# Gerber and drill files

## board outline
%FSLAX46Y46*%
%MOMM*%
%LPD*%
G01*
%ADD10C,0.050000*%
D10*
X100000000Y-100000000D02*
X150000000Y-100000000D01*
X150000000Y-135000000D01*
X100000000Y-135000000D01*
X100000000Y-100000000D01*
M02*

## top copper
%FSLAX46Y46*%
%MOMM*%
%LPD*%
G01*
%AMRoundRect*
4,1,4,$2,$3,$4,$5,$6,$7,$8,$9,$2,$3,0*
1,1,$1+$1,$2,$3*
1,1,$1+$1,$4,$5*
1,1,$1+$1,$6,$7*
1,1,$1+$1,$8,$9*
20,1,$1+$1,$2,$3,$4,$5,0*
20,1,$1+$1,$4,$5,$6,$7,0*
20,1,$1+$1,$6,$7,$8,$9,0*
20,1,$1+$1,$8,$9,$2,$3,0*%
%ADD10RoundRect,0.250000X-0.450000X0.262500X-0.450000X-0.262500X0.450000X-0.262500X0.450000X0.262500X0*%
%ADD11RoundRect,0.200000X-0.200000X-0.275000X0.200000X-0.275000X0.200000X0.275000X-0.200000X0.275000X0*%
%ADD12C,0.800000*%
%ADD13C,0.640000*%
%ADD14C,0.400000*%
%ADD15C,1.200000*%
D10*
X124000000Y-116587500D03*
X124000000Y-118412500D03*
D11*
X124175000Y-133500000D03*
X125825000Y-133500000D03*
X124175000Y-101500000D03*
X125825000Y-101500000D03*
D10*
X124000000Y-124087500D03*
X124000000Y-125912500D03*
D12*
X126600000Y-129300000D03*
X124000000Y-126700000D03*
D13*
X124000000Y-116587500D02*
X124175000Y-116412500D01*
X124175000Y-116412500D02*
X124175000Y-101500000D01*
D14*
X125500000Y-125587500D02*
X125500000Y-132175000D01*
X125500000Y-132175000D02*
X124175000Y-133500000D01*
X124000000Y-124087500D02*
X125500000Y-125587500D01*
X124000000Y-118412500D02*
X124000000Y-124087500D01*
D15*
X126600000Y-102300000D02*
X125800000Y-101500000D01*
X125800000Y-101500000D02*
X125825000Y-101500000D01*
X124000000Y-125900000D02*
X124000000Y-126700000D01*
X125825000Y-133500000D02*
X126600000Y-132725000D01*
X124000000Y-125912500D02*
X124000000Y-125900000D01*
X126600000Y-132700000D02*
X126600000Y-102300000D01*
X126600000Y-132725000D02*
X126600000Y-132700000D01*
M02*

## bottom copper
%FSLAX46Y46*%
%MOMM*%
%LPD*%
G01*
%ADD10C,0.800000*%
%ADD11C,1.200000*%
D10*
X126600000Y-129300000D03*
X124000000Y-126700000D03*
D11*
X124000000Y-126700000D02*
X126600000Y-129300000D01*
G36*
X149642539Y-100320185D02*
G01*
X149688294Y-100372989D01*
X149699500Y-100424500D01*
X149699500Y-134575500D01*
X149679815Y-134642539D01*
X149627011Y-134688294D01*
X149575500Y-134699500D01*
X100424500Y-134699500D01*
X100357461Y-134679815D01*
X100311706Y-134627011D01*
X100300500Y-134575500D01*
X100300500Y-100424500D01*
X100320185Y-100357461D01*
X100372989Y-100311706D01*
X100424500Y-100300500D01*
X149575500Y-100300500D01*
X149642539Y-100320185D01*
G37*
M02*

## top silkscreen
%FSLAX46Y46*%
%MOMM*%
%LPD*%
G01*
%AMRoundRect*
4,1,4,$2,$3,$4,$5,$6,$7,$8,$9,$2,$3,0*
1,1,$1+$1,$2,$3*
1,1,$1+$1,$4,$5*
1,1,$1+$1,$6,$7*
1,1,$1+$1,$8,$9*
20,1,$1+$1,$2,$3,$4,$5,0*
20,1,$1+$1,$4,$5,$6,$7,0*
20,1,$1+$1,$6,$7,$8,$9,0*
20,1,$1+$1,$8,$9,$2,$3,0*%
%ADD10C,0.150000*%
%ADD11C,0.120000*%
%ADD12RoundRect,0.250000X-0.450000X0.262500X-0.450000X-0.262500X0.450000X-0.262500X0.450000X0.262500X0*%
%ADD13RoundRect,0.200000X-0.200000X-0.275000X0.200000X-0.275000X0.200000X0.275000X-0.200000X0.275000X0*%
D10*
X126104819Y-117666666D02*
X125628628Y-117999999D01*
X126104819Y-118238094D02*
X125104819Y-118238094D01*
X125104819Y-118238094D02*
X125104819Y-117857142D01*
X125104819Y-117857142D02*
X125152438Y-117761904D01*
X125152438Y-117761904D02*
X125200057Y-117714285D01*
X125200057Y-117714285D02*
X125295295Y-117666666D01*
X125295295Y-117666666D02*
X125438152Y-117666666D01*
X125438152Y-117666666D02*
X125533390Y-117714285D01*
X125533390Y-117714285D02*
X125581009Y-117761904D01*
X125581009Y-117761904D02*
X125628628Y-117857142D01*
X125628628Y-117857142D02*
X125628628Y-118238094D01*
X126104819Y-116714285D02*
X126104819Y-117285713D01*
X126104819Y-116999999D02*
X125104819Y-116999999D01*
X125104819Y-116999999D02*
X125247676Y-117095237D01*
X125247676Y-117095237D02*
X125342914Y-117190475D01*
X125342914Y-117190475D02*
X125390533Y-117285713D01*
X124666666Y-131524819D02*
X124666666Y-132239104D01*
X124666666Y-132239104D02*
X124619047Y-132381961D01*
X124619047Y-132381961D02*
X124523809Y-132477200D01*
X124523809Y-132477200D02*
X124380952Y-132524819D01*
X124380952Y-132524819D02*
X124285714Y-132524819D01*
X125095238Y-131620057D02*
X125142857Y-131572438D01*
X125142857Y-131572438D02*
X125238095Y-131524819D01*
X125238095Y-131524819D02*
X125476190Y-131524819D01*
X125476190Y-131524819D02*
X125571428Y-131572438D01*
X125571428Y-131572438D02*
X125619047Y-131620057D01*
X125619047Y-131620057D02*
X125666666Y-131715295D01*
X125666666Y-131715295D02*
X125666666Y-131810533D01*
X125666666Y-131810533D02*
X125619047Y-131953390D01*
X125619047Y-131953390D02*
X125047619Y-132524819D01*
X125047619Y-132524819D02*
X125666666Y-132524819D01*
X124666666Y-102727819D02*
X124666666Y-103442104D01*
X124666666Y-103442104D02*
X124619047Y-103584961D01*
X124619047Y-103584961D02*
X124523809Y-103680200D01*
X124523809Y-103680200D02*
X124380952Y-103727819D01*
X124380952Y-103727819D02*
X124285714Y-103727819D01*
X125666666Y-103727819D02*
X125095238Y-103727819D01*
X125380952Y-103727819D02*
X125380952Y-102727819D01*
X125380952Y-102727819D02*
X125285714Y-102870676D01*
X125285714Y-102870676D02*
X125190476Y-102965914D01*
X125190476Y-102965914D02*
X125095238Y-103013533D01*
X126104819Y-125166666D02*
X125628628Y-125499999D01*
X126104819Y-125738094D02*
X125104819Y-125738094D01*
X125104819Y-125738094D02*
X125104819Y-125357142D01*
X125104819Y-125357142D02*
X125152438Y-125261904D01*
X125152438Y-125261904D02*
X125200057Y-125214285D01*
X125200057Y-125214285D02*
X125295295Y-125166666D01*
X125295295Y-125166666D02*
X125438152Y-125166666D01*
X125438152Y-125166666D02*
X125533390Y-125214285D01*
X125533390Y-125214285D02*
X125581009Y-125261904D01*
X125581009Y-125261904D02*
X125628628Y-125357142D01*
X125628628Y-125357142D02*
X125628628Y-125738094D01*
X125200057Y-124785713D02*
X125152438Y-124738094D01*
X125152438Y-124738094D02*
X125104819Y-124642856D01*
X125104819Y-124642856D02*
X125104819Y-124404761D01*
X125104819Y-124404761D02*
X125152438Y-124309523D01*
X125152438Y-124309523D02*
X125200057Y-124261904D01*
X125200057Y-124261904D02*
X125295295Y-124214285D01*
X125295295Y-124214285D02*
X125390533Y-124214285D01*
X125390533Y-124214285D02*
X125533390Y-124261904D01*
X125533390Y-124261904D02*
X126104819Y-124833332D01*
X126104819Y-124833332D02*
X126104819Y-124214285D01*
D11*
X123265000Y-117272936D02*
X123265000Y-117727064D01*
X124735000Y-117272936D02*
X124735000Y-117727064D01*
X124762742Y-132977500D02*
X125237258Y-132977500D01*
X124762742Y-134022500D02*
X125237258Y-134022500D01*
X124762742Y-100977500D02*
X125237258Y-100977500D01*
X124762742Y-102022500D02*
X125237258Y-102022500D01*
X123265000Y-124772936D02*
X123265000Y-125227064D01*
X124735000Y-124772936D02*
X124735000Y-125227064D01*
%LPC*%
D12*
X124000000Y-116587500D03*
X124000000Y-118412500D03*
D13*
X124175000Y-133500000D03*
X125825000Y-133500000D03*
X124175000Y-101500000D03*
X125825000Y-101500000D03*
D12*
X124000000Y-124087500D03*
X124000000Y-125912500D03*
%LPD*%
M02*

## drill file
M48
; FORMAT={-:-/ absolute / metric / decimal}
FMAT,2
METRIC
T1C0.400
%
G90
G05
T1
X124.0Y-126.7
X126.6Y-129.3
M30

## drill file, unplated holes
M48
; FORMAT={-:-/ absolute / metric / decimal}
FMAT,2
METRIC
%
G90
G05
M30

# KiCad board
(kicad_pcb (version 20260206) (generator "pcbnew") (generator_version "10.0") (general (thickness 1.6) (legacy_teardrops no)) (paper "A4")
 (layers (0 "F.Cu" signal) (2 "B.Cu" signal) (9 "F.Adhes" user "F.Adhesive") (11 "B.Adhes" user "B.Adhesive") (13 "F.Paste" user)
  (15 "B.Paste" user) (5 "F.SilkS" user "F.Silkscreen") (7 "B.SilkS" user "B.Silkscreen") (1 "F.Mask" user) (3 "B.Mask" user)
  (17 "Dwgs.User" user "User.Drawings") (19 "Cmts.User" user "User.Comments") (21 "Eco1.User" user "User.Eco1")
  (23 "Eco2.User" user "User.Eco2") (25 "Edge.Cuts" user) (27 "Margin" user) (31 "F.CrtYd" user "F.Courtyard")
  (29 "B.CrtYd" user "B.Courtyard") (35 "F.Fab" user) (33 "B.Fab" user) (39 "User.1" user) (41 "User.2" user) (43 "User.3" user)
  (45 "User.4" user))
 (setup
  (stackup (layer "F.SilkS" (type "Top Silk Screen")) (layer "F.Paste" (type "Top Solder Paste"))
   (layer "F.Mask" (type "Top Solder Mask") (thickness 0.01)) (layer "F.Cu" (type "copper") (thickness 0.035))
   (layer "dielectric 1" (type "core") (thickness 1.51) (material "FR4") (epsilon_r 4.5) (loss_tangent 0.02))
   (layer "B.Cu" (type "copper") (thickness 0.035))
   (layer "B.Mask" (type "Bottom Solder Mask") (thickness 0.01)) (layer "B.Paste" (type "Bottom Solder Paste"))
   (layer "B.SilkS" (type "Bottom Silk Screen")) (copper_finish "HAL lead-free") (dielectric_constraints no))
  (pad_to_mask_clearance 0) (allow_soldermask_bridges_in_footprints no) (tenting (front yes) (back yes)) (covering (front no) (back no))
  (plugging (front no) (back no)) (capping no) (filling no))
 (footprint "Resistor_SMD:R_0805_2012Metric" (layer "F.Cu") (at 124 117.5 -90)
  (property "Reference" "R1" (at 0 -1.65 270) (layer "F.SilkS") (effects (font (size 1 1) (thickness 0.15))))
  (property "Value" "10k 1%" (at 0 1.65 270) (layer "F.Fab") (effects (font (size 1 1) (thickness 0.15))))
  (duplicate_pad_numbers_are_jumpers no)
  (fp_line (start -0.227064 0.735) (end 0.227064 0.735) (stroke (width 0.12) (type solid)) (layer "F.SilkS"))
  (fp_line (start -0.227064 -0.735) (end 0.227064 -0.735) (stroke (width 0.12) (type solid)) (layer "F.SilkS"))
  (pad "1" smd roundrect (at -0.9125 0 270) (size 1.025 1.4) (layers "F.Cu" "F.Mask" "F.Paste") (roundrect_rratio 0.243902) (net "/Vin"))
  (pad "2" smd roundrect (at 0.9125 0 270) (size 1.025 1.4) (layers "F.Cu" "F.Mask" "F.Paste") (roundrect_rratio 0.243902) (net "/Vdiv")))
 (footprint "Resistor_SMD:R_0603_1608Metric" (layer "F.Cu") (at 125 133.5)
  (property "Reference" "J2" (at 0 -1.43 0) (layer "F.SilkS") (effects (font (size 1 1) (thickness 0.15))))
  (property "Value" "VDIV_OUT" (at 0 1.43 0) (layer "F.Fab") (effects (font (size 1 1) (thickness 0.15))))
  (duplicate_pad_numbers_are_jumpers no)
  (fp_line (start -0.237258 -0.5225) (end 0.237258 -0.5225) (stroke (width 0.12) (type solid)) (layer "F.SilkS"))
  (fp_line (start -0.237258 0.5225) (end 0.237258 0.5225) (stroke (width 0.12) (type solid)) (layer "F.SilkS"))
  (pad "1" smd roundrect (at -0.825 0) (size 0.8 0.95) (layers "F.Cu" "F.Mask" "F.Paste") (roundrect_rratio 0.25) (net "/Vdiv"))
  (pad "2" smd roundrect (at 0.825 0) (size 0.8 0.95) (layers "F.Cu" "F.Mask" "F.Paste") (roundrect_rratio 0.25) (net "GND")))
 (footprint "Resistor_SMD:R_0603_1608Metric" (layer "F.Cu") (at 125 101.5)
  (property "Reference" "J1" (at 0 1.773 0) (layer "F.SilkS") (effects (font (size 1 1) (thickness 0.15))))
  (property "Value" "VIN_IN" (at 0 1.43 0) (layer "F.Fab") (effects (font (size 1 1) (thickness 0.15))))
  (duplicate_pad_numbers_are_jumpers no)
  (fp_line (start -0.237258 -0.5225) (end 0.237258 -0.5225) (stroke (width 0.12) (type solid)) (layer "F.SilkS"))
  (fp_line (start -0.237258 0.5225) (end 0.237258 0.5225) (stroke (width 0.12) (type solid)) (layer "F.SilkS"))
  (pad "1" smd roundrect (at -0.825 0) (size 0.8 0.95) (layers "F.Cu" "F.Mask" "F.Paste") (roundrect_rratio 0.25) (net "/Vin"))
  (pad "2" smd roundrect (at 0.825 0) (size 0.8 0.95) (layers "F.Cu" "F.Mask" "F.Paste") (roundrect_rratio 0.25) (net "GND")))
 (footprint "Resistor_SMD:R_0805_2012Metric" (layer "F.Cu") (at 124 125 -90)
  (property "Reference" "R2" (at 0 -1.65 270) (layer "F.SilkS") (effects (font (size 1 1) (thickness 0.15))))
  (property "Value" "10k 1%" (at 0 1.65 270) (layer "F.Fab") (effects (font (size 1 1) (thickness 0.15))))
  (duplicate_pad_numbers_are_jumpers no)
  (fp_line (start -0.227064 0.735) (end 0.227064 0.735) (stroke (width 0.12) (type solid)) (layer "F.SilkS"))
  (fp_line (start -0.227064 -0.735) (end 0.227064 -0.735) (stroke (width 0.12) (type solid)) (layer "F.SilkS"))
  (pad "1" smd roundrect (at -0.9125 0 270) (size 1.025 1.4) (layers "F.Cu" "F.Mask" "F.Paste") (roundrect_rratio 0.243902) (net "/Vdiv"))
  (pad "2" smd roundrect (at 0.9125 0 270) (size 1.025 1.4) (layers "F.Cu" "F.Mask" "F.Paste") (roundrect_rratio 0.243902) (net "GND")))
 (gr_rect (start 100 100) (end 150 135) (stroke (width 0.05) (type solid)) (fill no) (layer "Edge.Cuts"))
 (segment (start 124 116.5875) (end 124.175 116.4125) (width 0.64) (layer "F.Cu") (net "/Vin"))
 (segment (start 124.175 116.4125) (end 124.175 101.5) (width 0.64) (layer "F.Cu") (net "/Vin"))
 (segment (start 125.5 125.5875) (end 125.5 132.175) (width 0.4) (layer "F.Cu") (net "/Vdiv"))
 (segment (start 125.5 132.175) (end 124.175 133.5) (width 0.4) (layer "F.Cu") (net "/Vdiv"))
 (segment (start 124 124.0875) (end 125.5 125.5875) (width 0.4) (layer "F.Cu") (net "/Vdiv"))
 (segment (start 124 118.4125) (end 124 124.0875) (width 0.4) (layer "F.Cu") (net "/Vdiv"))
 (segment (start 126.6 102.3) (end 125.8 101.5) (width 1.2) (layer "F.Cu") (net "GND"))
 (segment (start 125.8 101.5) (end 125.825 101.5) (width 1.2) (layer "F.Cu") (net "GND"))
 (segment (start 124 125.9) (end 124 126.7) (width 1.2) (layer "F.Cu") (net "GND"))
 (segment (start 125.825 133.5) (end 126.6 132.725) (width 1.2) (layer "F.Cu") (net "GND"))
 (segment (start 124 125.9125) (end 124 125.9) (width 1.2) (layer "F.Cu") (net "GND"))
 (segment (start 126.6 132.7) (end 126.6 102.3) (width 1.2) (layer "F.Cu") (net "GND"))
 (segment (start 126.6 132.725) (end 126.6 132.7) (width 1.2) (layer "F.Cu") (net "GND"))
 (via (at 126.6 129.3) (size 0.8) (drill 0.4) (layers "F.Cu" "B.Cu") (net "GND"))
 (via (at 124 126.7) (size 0.8) (drill 0.4) (layers "F.Cu" "B.Cu") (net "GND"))
 (segment (start 124 126.7) (end 126.6 129.3) (width 1.2) (layer "B.Cu") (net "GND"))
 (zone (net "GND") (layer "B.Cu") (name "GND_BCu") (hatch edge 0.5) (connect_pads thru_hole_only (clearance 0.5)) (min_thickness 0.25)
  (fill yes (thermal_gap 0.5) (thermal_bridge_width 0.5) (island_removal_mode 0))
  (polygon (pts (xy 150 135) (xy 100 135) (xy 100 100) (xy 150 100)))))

